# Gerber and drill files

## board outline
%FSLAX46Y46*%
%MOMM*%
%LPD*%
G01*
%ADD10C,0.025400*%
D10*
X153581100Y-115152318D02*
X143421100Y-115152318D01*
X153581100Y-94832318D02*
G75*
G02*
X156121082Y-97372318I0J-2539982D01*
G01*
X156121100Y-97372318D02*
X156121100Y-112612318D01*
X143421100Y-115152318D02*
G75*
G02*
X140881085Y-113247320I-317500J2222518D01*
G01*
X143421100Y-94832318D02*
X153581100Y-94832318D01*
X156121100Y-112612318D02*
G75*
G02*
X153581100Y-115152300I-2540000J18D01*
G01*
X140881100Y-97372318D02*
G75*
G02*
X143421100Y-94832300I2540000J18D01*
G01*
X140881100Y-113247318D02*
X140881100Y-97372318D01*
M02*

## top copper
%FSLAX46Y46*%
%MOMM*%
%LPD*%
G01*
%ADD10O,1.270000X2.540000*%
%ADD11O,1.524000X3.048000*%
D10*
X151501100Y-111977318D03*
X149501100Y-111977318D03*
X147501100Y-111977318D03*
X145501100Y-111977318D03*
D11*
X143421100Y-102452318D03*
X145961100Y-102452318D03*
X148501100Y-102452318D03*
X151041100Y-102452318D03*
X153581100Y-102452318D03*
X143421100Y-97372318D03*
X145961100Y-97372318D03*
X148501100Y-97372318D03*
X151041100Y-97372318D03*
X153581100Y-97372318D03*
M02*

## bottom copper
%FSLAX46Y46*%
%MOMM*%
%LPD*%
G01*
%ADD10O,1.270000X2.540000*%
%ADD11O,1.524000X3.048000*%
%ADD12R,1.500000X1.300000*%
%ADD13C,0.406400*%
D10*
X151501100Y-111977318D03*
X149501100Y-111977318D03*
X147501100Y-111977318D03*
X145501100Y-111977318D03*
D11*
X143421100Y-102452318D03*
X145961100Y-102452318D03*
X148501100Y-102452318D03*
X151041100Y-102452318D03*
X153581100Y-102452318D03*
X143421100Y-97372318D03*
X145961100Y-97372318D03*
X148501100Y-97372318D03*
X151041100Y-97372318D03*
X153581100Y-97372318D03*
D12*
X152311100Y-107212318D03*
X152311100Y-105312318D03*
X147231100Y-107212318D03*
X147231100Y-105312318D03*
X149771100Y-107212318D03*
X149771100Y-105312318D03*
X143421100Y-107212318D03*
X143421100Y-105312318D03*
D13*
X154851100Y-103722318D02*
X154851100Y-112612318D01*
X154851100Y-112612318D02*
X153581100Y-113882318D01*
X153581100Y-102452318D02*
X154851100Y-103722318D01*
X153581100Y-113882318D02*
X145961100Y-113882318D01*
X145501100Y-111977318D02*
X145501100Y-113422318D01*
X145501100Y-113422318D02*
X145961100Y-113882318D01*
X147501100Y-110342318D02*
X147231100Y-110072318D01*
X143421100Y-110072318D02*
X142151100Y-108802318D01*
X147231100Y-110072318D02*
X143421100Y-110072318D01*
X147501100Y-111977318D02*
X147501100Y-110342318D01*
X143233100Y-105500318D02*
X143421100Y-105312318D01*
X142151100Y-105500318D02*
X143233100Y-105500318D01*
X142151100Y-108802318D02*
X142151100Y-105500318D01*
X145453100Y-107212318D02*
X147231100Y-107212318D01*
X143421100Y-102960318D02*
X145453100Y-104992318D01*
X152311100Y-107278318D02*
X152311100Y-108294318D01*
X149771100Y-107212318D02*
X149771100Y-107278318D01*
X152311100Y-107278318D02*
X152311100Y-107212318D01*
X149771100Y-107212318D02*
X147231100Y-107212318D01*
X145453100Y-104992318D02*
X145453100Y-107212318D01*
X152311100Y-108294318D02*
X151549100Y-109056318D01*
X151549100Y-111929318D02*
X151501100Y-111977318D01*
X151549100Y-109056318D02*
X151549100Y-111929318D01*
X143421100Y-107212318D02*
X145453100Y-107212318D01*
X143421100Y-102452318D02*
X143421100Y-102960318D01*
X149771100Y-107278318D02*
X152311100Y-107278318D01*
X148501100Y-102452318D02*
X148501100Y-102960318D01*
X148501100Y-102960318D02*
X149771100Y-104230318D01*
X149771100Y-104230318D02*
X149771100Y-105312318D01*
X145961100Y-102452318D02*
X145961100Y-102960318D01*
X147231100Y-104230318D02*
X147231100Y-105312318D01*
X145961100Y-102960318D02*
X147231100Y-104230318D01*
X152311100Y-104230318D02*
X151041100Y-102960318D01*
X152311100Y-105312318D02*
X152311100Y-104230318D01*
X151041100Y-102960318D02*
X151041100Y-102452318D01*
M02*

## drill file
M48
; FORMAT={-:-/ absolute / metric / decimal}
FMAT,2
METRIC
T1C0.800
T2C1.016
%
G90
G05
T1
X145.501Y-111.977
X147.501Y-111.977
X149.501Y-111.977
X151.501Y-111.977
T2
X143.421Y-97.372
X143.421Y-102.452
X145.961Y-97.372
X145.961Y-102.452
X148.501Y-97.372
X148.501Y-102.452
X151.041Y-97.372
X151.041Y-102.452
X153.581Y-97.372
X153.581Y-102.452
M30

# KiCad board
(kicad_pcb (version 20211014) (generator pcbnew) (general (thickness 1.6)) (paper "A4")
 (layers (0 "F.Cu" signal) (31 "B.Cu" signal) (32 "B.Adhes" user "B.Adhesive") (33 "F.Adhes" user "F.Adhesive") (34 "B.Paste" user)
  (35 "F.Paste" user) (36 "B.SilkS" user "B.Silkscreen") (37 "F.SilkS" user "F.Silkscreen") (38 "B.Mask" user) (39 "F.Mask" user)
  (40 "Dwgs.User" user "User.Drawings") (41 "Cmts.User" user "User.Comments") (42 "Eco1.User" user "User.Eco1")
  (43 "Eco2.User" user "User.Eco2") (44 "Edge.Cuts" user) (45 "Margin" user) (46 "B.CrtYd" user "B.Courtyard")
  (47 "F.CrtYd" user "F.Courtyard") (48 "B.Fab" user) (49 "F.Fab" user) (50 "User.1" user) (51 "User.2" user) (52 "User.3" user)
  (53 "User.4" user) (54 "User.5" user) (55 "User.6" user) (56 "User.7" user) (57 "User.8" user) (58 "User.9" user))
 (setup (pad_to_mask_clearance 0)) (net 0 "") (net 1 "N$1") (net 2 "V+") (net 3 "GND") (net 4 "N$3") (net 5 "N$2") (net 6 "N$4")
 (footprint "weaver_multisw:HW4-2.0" (layer "F.Cu") (at 148.5011 111.977318 180)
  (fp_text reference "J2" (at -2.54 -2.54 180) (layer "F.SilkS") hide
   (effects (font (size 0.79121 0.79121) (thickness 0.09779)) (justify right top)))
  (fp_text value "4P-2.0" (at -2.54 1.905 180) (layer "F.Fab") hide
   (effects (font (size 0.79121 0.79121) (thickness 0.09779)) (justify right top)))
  (pad "1" thru_hole oval (at -3 0 270) (size 2.54 1.27) (drill 0.8) (layers *.Cu *.Mask) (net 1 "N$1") (solder_mask_margin 0.0508))
  (pad "2" thru_hole oval (at -1 0 270) (size 2.54 1.27) (drill 0.8) (layers *.Cu *.Mask) (solder_mask_margin 0.0508))
  (pad "3" thru_hole oval (at 1 0 270) (size 2.54 1.27) (drill 0.8) (layers *.Cu *.Mask) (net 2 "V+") (solder_mask_margin 0.0508))
  (pad "4" thru_hole oval (at 3 0 270) (size 2.54 1.27) (drill 0.8) (layers *.Cu *.Mask) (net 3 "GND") (solder_mask_margin 0.0508)))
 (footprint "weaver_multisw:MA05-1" (layer "F.Cu") (at 148.5011 102.452318)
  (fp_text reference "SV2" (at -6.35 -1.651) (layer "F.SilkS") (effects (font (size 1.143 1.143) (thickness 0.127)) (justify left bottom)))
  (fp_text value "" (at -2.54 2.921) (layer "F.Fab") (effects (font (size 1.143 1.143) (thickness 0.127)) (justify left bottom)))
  (pad "1" thru_hole oval (at -5.08 0 90) (size 3.048 1.524) (drill 1.016) (layers *.Cu *.Mask) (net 1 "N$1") (solder_mask_margin 0.0508))
  (pad "2" thru_hole oval (at -2.54 0 90) (size 3.048 1.524) (drill 1.016) (layers *.Cu *.Mask) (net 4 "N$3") (solder_mask_margin 0.0508))
  (pad "3" thru_hole oval (at 0 0 90) (size 3.048 1.524) (drill 1.016) (layers *.Cu *.Mask) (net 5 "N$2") (solder_mask_margin 0.0508))
  (pad "4" thru_hole oval (at 2.54 0 90) (size 3.048 1.524) (drill 1.016) (layers *.Cu *.Mask) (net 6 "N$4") (solder_mask_margin 0.0508))
  (pad "5" thru_hole oval (at 5.08 0 90) (size 3.048 1.524) (drill 1.016) (layers *.Cu *.Mask) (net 3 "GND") (solder_mask_margin 0.0508)))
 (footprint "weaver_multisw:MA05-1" (layer "F.Cu") (at 148.5011 97.372318)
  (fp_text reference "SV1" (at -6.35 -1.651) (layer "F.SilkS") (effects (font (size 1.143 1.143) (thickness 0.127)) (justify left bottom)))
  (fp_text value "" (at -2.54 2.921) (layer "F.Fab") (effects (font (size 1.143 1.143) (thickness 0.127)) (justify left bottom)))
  (pad "1" thru_hole oval (at -5.08 0 90) (size 3.048 1.524) (drill 1.016) (layers *.Cu *.Mask) (solder_mask_margin 0.0508))
  (pad "2" thru_hole oval (at -2.54 0 90) (size 3.048 1.524) (drill 1.016) (layers *.Cu *.Mask) (solder_mask_margin 0.0508))
  (pad "3" thru_hole oval (at 0 0 90) (size 3.048 1.524) (drill 1.016) (layers *.Cu *.Mask) (solder_mask_margin 0.0508))
  (pad "4" thru_hole oval (at 2.54 0 90) (size 3.048 1.524) (drill 1.016) (layers *.Cu *.Mask) (solder_mask_margin 0.0508))
  (pad "5" thru_hole oval (at 5.08 0 90) (size 3.048 1.524) (drill 1.016) (layers *.Cu *.Mask) (solder_mask_margin 0.0508)))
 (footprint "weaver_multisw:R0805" (layer "B.Cu") (at 152.3111 106.262318 90)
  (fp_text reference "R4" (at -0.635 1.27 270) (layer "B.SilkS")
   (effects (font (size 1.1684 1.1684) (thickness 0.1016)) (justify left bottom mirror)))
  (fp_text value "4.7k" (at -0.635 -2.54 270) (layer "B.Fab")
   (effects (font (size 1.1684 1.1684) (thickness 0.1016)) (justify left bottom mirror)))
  (pad "1" smd rect (at -0.95 0 90) (size 1.3 1.5) (layers "B.Cu" "B.Paste" "B.Mask") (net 1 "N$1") (solder_mask_margin 0.0508))
  (pad "2" smd rect (at 0.95 0 90) (size 1.3 1.5) (layers "B.Cu" "B.Paste" "B.Mask") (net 6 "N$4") (solder_mask_margin 0.0508)))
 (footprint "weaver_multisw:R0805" (layer "B.Cu") (at 147.2311 106.262318 90)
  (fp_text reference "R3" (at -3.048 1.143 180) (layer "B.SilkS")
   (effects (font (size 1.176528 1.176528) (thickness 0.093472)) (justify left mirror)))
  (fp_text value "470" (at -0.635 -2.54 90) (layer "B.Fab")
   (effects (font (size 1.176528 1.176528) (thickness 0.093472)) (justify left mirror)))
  (pad "1" smd rect (at -0.95 0 90) (size 1.3 1.5) (layers "B.Cu" "B.Paste" "B.Mask") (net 1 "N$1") (solder_mask_margin 0.0508))
  (pad "2" smd rect (at 0.95 0 90) (size 1.3 1.5) (layers "B.Cu" "B.Paste" "B.Mask") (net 4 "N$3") (solder_mask_margin 0.0508)))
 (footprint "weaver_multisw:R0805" (layer "B.Cu") (at 149.7711 106.262318 90)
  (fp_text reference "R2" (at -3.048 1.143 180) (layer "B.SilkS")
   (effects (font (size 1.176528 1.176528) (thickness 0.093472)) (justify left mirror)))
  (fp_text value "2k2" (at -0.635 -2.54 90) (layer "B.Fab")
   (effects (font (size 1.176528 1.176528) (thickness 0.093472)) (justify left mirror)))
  (pad "1" smd rect (at -0.95 0 90) (size 1.3 1.5) (layers "B.Cu" "B.Paste" "B.Mask") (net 1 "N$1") (solder_mask_margin 0.0508))
  (pad "2" smd rect (at 0.95 0 90) (size 1.3 1.5) (layers "B.Cu" "B.Paste" "B.Mask") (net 5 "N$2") (solder_mask_margin 0.0508)))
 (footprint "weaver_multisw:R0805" (layer "B.Cu") (at 143.4211 106.262318 90)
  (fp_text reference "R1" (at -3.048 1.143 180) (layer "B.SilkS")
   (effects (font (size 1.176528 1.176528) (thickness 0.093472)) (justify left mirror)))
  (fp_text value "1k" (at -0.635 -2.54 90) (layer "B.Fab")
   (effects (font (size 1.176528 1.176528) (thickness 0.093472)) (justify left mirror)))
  (pad "1" smd rect (at -0.95 0 90) (size 1.3 1.5) (layers "B.Cu" "B.Paste" "B.Mask") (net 1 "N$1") (solder_mask_margin 0.0508))
  (pad "2" smd rect (at 0.95 0 90) (size 1.3 1.5) (layers "B.Cu" "B.Paste" "B.Mask") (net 2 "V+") (solder_mask_margin 0.0508)))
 (gr_line (start 153.5811 115.152318) (end 143.4211 115.152318) (layer "Edge.Cuts") (width 0.0254))
 (gr_arc (start 153.5811 94.832318) (mid 155.377151 95.576267) (end 156.1211 97.372318) (layer "Edge.Cuts") (width 0.0254))
 (gr_line (start 156.1211 97.372318) (end 156.1211 112.612318) (layer "Edge.Cuts") (width 0.0254))
 (gr_arc (start 143.4211 115.152318) (mid 141.756562 114.725869) (end 140.8811 113.247318) (layer "Edge.Cuts") (width 0.0254))
 (gr_line (start 143.4211 94.832318) (end 153.5811 94.832318) (layer "Edge.Cuts") (width 0.0254))
 (gr_arc (start 156.1211 112.612318) (mid 155.377151 114.408369) (end 153.5811 115.152318) (layer "Edge.Cuts") (width 0.0254))
 (gr_arc (start 140.8811 97.372318) (mid 141.625049 95.576267) (end 143.4211 94.832318) (layer "Edge.Cuts") (width 0.0254))
 (gr_line (start 140.8811 113.247318) (end 140.8811 97.372318) (layer "Edge.Cuts") (width 0.0254))
 (segment (start 154.8511 103.722318) (end 154.8511 112.612318) (width 0.4064) (layer "B.Cu") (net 3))
 (segment (start 154.8511 112.612318) (end 153.5811 113.882318) (width 0.4064) (layer "B.Cu") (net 3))
 (segment (start 153.5811 102.452318) (end 154.8511 103.722318) (width 0.4064) (layer "B.Cu") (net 3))
 (segment (start 153.5811 113.882318) (end 145.9611 113.882318) (width 0.4064) (layer "B.Cu") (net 3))
 (segment (start 145.5011 111.977318) (end 145.5011 113.422318) (width 0.4064) (layer "B.Cu") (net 3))
 (segment (start 145.5011 113.422318) (end 145.9611 113.882318) (width 0.4064) (layer "B.Cu") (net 3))
 (segment (start 147.5011 110.342318) (end 147.2311 110.072318) (width 0.4064) (layer "B.Cu") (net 2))
 (segment (start 143.4211 110.072318) (end 142.1511 108.802318) (width 0.4064) (layer "B.Cu") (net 2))
 (segment (start 147.2311 110.072318) (end 143.4211 110.072318) (width 0.4064) (layer "B.Cu") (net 2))
 (segment (start 147.5011 111.977318) (end 147.5011 110.342318) (width 0.4064) (layer "B.Cu") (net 2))
 (segment (start 143.2331 105.500318) (end 143.4211 105.312318) (width 0.4064) (layer "B.Cu") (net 2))
 (segment (start 142.1511 105.500318) (end 143.2331 105.500318) (width 0.4064) (layer "B.Cu") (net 2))
 (segment (start 142.1511 108.802318) (end 142.1511 105.500318) (width 0.4064) (layer "B.Cu") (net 2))
 (segment (start 145.4531 107.212318) (end 147.2311 107.212318) (width 0.4064) (layer "B.Cu") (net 1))
 (segment (start 143.4211 102.960318) (end 145.4531 104.992318) (width 0.4064) (layer "B.Cu") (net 1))
 (segment (start 152.3111 107.278318) (end 152.3111 108.294318) (width 0.4064) (layer "B.Cu") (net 1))
 (segment (start 149.7711 107.212318) (end 149.7711 107.278318) (width 0.4064) (layer "B.Cu") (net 1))
 (segment (start 152.3111 107.278318) (end 152.3111 107.212318) (width 0.4064) (layer "B.Cu") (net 1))
 (segment (start 149.7711 107.212318) (end 147.2311 107.212318) (width 0.4064) (layer "B.Cu") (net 1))
 (segment (start 145.4531 104.992318) (end 145.4531 107.212318) (width 0.4064) (layer "B.Cu") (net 1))
 (segment (start 152.3111 108.294318) (end 151.5491 109.056318) (width 0.4064) (layer "B.Cu") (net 1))
 (segment (start 151.5491 111.929318) (end 151.5011 111.977318) (width 0.4064) (layer "B.Cu") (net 1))
 (segment (start 151.5491 109.056318) (end 151.5491 111.929318) (width 0.4064) (layer "B.Cu") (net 1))
 (segment (start 143.4211 107.212318) (end 145.4531 107.212318) (width 0.4064) (layer "B.Cu") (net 1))
 (segment (start 143.4211 102.452318) (end 143.4211 102.960318) (width 0.4064) (layer "B.Cu") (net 1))
 (segment (start 149.7711 107.278318) (end 152.3111 107.278318) (width 0.4064) (layer "B.Cu") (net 1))
 (segment (start 148.5011 102.452318) (end 148.5011 102.960318) (width 0.4064) (layer "B.Cu") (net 5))
 (segment (start 148.5011 102.960318) (end 149.7711 104.230318) (width 0.4064) (layer "B.Cu") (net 5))
 (segment (start 149.7711 104.230318) (end 149.7711 105.312318) (width 0.4064) (layer "B.Cu") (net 5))
 (segment (start 145.9611 102.452318) (end 145.9611 102.960318) (width 0.4064) (layer "B.Cu") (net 4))
 (segment (start 147.2311 104.230318) (end 147.2311 105.312318) (width 0.4064) (layer "B.Cu") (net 4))
 (segment (start 145.9611 102.960318) (end 147.2311 104.230318) (width 0.4064) (layer "B.Cu") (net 4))
 (segment (start 152.3111 104.230318) (end 151.0411 102.960318) (width 0.4064) (layer "B.Cu") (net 6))
 (segment (start 152.3111 105.312318) (end 152.3111 104.230318) (width 0.4064) (layer "B.Cu") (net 6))
 (segment (start 151.0411 102.960318) (end 151.0411 102.452318) (width 0.4064) (layer "B.Cu") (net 6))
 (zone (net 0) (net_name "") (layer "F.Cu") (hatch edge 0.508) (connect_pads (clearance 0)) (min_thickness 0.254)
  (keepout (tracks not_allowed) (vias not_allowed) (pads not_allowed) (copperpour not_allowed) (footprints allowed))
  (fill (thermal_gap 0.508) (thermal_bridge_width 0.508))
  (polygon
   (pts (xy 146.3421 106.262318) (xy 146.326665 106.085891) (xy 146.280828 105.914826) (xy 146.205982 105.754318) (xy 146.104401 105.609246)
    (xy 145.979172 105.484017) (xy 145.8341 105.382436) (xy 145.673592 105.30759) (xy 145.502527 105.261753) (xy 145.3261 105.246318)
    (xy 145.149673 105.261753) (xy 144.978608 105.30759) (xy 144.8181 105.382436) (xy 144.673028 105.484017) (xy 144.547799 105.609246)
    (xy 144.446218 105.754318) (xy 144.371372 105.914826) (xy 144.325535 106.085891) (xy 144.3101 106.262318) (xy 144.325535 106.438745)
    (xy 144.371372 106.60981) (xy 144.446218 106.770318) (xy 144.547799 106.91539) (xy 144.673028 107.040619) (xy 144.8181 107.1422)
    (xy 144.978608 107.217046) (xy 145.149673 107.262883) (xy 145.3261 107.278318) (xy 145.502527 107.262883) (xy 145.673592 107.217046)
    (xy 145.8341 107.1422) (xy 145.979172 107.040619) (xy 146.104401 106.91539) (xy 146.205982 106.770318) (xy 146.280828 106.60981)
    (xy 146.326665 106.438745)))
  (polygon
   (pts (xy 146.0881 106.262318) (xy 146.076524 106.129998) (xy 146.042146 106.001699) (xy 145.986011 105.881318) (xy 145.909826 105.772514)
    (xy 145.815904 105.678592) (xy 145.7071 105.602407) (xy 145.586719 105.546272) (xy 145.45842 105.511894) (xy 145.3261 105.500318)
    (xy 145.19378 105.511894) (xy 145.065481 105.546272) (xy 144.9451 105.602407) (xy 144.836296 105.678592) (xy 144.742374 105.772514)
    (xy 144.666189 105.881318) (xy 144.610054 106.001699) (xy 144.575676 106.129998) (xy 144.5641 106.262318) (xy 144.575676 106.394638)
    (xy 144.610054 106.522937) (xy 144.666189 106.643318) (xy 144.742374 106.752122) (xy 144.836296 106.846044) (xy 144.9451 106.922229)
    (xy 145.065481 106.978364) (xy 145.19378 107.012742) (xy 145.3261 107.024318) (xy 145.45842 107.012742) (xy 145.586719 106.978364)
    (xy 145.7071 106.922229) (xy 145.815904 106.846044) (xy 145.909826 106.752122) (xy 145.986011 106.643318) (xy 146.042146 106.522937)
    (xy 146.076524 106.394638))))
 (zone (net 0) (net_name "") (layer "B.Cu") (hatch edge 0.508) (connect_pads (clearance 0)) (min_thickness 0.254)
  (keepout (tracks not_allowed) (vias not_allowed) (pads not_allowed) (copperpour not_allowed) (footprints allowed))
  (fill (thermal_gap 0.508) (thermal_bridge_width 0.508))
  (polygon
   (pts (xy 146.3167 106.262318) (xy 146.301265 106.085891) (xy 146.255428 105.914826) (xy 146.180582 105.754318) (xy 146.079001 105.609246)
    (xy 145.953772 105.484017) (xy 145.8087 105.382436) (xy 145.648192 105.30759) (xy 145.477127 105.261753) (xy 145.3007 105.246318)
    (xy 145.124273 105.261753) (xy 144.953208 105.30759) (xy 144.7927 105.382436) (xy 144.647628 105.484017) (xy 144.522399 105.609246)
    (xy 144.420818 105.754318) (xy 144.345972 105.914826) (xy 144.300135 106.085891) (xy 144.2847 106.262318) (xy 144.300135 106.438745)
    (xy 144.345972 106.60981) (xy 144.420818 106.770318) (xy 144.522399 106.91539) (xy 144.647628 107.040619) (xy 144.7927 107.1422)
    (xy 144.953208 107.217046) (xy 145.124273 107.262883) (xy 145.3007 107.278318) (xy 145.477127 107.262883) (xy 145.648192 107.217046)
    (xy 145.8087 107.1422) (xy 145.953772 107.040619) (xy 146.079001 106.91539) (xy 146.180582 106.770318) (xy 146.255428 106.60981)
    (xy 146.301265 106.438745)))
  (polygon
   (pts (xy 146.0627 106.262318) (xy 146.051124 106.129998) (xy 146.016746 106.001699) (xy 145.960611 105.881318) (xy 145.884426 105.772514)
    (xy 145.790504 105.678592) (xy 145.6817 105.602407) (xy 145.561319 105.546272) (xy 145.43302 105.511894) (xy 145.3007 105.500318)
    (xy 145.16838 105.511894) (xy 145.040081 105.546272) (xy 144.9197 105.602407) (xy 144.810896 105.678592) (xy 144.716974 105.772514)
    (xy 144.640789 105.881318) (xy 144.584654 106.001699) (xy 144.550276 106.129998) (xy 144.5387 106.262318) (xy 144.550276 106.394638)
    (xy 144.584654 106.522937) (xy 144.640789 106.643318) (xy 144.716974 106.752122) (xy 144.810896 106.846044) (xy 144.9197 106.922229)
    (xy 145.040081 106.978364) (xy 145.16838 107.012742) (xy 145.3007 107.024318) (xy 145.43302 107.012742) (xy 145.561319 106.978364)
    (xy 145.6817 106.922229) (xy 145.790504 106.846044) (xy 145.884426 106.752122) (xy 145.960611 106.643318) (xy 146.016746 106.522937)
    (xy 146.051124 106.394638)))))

